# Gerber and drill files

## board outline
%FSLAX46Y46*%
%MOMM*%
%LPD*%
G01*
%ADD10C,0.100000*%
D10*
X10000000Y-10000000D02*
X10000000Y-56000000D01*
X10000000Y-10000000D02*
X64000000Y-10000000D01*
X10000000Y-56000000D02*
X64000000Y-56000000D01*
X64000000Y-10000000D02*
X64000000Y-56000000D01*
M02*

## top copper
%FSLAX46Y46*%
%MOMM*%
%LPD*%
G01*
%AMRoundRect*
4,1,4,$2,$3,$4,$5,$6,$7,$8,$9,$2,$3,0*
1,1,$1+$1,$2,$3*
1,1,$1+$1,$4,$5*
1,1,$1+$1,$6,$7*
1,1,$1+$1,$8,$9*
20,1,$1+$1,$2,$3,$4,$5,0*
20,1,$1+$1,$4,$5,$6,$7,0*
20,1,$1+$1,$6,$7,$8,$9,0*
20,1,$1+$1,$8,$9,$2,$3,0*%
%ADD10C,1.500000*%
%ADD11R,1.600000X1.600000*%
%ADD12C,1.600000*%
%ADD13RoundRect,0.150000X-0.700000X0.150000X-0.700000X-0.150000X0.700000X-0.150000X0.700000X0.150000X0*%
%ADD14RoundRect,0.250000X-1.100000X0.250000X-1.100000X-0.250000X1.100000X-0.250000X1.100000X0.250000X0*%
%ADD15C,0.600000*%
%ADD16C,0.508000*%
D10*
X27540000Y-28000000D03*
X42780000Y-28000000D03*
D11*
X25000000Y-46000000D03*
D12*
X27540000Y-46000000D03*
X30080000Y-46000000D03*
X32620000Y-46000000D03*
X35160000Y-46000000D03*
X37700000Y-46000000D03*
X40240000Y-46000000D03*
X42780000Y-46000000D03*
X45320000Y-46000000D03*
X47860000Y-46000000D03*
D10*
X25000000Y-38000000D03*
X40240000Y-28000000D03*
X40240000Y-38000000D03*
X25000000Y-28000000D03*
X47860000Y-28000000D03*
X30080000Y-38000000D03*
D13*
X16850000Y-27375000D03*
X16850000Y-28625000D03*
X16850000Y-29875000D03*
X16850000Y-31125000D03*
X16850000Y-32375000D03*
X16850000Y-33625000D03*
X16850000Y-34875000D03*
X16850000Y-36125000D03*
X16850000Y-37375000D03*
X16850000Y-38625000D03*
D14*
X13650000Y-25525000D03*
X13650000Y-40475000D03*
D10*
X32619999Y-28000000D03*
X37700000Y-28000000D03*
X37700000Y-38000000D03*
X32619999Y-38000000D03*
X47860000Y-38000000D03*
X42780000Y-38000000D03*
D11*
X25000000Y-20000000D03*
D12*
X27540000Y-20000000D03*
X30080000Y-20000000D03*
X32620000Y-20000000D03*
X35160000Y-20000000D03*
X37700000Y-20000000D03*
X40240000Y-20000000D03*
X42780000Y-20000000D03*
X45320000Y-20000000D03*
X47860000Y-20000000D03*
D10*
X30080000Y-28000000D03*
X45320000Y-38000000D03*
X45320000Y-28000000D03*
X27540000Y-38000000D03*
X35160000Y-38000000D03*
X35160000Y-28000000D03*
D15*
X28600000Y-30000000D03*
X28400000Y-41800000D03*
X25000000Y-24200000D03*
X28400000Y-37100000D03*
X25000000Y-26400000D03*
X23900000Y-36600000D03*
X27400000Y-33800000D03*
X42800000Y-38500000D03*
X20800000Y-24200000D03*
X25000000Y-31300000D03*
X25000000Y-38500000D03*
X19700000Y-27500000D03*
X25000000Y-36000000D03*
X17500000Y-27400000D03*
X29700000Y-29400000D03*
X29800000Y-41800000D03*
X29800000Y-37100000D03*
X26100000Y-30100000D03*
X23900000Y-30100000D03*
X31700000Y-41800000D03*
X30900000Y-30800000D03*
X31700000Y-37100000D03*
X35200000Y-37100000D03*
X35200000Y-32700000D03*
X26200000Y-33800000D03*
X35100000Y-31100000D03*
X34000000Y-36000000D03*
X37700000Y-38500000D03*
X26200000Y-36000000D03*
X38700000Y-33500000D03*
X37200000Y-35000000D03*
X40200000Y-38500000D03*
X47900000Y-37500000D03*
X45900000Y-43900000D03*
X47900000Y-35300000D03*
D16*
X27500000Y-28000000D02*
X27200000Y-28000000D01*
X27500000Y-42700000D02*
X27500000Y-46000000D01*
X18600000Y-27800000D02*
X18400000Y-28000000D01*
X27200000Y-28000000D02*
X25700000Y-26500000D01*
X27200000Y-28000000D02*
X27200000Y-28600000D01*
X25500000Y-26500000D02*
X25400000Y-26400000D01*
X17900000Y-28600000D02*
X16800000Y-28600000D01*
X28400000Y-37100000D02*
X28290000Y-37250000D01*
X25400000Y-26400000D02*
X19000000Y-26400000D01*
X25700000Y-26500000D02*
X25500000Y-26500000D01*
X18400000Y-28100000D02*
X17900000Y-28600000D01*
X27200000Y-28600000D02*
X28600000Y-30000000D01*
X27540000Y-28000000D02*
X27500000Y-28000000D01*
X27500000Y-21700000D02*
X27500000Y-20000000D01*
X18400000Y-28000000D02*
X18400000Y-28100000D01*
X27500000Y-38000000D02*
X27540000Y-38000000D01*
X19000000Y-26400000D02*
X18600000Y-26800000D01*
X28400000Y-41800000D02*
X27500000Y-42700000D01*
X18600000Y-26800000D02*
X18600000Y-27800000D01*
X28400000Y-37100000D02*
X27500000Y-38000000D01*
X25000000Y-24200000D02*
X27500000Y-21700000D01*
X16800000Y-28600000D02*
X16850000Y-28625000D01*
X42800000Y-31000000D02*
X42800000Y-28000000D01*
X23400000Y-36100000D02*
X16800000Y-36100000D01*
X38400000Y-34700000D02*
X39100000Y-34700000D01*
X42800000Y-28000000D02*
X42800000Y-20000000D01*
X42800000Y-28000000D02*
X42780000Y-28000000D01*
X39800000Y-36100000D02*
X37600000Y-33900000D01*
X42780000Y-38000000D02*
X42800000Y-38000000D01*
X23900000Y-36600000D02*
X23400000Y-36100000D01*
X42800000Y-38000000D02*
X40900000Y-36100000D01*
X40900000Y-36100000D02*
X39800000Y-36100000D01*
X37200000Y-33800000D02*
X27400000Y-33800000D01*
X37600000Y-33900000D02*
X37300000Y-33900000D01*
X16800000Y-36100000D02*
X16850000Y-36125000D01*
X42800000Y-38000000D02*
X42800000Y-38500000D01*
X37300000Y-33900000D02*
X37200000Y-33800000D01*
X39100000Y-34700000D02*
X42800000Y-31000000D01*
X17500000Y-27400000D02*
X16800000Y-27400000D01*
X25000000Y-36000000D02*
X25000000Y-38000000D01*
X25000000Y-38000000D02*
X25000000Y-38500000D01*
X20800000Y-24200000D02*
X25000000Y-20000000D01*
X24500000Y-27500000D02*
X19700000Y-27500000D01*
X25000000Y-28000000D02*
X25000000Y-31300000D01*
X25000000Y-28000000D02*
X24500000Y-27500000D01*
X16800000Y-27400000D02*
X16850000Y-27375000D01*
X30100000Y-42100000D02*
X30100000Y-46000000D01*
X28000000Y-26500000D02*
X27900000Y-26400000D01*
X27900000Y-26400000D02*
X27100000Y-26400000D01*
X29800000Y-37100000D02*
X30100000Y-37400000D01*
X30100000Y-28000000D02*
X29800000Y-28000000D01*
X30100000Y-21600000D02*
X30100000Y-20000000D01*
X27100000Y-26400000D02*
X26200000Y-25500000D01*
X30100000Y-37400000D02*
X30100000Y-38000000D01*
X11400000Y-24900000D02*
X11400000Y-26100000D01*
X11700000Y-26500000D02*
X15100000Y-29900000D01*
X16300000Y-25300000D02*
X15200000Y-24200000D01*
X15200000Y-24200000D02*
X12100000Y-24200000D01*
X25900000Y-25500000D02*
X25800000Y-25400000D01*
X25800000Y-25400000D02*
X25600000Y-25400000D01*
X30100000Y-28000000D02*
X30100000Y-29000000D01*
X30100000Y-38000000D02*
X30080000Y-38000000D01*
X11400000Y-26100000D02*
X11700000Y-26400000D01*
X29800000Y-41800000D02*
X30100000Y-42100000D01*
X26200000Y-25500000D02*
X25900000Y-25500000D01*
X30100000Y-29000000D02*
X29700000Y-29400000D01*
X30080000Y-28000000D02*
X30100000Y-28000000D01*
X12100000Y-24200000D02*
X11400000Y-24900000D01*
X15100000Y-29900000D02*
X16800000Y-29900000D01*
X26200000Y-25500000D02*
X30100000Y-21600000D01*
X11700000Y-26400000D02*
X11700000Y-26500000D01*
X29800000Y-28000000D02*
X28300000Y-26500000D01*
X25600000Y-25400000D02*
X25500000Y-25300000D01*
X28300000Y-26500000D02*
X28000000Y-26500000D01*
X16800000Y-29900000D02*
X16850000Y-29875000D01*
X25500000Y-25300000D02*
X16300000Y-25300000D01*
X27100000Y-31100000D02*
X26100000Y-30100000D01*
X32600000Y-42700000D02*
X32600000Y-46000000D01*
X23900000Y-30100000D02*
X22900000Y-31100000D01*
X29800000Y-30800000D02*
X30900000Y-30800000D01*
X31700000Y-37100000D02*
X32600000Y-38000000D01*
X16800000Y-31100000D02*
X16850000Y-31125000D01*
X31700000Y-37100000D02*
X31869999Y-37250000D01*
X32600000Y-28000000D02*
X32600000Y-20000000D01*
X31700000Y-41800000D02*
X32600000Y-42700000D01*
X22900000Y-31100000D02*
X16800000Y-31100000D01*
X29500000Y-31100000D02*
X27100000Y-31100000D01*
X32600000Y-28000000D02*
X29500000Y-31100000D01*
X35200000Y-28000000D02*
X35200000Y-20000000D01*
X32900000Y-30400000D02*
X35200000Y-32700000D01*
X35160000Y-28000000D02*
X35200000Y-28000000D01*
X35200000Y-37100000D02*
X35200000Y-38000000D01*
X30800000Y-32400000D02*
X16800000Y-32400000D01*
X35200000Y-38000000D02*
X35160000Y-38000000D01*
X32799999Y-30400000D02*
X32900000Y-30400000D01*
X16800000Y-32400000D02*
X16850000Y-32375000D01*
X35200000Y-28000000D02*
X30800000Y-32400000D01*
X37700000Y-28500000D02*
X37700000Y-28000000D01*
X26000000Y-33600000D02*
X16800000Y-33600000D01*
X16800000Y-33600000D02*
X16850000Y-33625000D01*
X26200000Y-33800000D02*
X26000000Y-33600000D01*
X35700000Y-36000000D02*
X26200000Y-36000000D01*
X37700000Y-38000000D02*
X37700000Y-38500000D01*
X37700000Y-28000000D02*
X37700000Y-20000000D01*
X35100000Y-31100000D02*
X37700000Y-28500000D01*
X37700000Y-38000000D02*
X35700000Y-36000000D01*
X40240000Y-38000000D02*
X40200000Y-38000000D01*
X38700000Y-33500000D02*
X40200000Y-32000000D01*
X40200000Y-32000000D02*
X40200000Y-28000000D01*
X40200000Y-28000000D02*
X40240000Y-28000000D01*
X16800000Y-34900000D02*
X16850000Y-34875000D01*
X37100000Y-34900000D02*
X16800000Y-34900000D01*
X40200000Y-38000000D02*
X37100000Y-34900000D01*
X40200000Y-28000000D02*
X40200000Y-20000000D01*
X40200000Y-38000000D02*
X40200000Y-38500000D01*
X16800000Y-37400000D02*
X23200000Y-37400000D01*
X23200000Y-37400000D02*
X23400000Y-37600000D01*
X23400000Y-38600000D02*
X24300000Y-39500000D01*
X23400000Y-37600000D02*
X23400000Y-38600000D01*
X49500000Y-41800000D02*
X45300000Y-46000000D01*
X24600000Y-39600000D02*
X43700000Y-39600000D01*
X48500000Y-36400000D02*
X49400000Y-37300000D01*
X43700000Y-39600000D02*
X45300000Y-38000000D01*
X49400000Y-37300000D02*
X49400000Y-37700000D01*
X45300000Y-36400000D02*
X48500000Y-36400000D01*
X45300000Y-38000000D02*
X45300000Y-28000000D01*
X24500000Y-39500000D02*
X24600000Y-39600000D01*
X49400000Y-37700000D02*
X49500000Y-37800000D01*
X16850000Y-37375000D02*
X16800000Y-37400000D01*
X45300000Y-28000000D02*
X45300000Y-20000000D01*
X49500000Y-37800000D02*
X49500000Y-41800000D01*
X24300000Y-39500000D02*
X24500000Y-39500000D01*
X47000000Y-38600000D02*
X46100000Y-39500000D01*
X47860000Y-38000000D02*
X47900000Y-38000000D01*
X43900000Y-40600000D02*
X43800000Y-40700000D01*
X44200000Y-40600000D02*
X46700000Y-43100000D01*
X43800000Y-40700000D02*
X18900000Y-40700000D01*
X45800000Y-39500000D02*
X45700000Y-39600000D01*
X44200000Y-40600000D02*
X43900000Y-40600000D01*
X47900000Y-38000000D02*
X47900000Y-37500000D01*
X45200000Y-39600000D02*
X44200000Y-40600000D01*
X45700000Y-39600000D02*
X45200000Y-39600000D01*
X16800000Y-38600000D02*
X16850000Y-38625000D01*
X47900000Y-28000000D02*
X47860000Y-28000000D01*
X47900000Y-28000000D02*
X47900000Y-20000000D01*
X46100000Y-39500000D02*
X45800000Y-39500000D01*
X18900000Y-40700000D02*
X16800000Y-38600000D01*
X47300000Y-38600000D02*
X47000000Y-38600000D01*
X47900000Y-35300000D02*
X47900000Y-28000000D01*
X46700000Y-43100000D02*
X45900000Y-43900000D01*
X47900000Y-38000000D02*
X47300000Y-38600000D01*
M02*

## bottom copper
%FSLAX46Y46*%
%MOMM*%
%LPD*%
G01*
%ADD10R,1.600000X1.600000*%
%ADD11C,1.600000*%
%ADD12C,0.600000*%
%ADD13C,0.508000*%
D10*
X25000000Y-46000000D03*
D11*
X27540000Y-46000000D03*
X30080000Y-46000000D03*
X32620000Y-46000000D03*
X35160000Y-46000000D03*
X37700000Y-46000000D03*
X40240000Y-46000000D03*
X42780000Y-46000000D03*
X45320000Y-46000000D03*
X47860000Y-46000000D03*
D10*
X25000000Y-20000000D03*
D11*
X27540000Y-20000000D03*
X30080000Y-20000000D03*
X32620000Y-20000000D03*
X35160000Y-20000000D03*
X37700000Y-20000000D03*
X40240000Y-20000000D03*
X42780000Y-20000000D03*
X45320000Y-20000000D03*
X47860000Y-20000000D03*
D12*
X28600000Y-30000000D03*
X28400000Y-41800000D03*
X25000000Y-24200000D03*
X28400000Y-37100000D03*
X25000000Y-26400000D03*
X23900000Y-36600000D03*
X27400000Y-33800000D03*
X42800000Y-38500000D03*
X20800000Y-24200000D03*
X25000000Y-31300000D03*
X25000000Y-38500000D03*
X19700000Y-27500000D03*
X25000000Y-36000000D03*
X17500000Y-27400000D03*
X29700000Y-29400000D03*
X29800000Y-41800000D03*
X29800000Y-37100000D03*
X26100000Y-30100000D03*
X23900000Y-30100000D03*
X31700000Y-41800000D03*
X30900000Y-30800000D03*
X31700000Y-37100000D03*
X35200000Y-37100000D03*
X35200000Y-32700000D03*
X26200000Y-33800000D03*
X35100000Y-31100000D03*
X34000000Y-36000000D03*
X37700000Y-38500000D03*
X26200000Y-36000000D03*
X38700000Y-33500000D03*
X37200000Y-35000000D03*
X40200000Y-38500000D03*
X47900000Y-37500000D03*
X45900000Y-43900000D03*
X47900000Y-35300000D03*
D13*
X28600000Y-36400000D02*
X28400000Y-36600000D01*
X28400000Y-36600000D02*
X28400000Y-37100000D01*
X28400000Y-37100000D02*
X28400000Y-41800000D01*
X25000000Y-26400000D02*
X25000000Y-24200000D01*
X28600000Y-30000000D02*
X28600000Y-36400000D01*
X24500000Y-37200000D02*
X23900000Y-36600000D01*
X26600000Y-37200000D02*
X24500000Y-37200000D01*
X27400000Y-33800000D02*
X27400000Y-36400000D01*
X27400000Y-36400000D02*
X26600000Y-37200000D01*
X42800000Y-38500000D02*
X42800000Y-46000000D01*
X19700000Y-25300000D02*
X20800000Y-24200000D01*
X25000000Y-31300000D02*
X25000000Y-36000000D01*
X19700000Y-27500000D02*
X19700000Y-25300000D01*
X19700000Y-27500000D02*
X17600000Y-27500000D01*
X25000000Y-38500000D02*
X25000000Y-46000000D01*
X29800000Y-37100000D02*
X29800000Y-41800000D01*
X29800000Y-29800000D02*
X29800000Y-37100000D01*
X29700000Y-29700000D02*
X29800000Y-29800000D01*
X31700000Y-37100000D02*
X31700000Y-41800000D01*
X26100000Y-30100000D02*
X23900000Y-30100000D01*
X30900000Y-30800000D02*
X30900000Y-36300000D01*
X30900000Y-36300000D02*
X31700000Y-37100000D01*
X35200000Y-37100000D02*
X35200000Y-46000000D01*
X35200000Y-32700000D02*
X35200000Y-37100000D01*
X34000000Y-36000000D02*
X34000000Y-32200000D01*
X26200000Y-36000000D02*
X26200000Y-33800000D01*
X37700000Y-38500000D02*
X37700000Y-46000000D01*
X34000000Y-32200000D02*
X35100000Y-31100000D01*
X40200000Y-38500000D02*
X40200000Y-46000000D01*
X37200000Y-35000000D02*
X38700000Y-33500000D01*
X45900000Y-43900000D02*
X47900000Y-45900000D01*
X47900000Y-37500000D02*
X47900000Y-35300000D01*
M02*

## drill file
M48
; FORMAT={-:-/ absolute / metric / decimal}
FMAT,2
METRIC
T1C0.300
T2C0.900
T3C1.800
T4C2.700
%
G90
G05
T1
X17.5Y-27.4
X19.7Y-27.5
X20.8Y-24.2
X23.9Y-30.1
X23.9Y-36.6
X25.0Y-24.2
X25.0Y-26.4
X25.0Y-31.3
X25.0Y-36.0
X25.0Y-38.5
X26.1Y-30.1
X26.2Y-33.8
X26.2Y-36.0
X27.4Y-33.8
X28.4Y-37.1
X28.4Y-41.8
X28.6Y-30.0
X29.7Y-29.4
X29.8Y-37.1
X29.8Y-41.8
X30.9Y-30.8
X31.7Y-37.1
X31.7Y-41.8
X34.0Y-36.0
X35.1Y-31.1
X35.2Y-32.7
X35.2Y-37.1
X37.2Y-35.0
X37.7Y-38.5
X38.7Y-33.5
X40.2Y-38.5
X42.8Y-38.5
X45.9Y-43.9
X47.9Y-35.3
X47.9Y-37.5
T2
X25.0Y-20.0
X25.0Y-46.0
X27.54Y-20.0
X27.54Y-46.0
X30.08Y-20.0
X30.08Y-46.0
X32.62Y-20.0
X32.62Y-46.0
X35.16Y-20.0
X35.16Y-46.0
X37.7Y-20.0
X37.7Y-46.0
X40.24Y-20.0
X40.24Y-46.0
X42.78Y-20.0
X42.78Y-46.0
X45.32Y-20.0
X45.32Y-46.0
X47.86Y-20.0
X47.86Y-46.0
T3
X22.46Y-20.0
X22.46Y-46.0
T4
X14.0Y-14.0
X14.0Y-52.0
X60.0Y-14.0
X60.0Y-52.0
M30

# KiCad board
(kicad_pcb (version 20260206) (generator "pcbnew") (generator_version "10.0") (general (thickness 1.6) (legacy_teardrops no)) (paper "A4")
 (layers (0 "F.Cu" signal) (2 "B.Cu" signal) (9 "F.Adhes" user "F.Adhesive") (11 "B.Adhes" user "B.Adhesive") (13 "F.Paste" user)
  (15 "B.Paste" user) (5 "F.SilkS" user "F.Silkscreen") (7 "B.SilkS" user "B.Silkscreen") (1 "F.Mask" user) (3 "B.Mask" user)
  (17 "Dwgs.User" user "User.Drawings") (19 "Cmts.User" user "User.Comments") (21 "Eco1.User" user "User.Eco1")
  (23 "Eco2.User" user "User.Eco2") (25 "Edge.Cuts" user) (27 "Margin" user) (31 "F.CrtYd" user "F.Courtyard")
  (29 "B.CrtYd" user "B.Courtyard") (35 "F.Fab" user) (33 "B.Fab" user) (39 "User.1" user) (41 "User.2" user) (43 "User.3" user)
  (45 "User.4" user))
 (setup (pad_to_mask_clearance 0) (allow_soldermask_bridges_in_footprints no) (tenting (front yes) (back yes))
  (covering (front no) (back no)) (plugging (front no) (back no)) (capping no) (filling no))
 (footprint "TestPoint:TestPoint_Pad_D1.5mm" (layer "F.Cu") (at 27.54 28)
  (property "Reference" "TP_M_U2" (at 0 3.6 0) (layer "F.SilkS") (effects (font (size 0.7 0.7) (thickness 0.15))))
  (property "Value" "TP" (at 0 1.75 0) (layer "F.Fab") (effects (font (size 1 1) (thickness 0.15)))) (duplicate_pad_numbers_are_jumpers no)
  (pad "1" smd circle (at 0 0) (size 1.5 1.5) (layers "F.Cu" "F.Mask") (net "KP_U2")))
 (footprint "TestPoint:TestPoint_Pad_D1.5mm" (layer "F.Cu") (at 42.78 28)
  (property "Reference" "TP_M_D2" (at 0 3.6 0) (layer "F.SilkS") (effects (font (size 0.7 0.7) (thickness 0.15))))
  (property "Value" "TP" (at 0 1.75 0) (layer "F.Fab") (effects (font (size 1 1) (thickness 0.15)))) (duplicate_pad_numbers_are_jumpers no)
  (pad "1" smd circle (at 0 0) (size 1.5 1.5) (layers "F.Cu" "F.Mask") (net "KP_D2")))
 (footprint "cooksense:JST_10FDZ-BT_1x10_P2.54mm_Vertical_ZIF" (layer "F.Cu") (at 25 46)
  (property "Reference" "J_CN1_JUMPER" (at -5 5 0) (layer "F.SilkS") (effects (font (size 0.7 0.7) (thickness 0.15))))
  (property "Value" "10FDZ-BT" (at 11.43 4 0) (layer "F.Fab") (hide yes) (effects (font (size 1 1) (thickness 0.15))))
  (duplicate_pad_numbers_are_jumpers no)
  (pad "" np_thru_hole circle (at -2.54 0) (size 1.8 1.8) (drill 1.8) (layers "*.Cu" "*.Mask"))
  (pad "1" thru_hole rect (at 0 0) (size 1.6 1.6) (drill 0.9) (layers "*.Cu" "*.Mask") (remove_unused_layers no) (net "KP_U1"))
  (pad "2" thru_hole circle (at 2.54 0) (size 1.6 1.6) (drill 0.9) (layers "*.Cu" "*.Mask") (remove_unused_layers no) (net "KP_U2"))
  (pad "3" thru_hole circle (at 5.08 0) (size 1.6 1.6) (drill 0.9) (layers "*.Cu" "*.Mask") (remove_unused_layers no) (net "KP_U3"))
  (pad "4" thru_hole circle (at 7.62 0) (size 1.6 1.6) (drill 0.9) (layers "*.Cu" "*.Mask") (remove_unused_layers no) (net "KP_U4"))
  (pad "5" thru_hole circle (at 10.16 0) (size 1.6 1.6) (drill 0.9) (layers "*.Cu" "*.Mask") (remove_unused_layers no) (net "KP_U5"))
  (pad "6" thru_hole circle (at 12.7 0) (size 1.6 1.6) (drill 0.9) (layers "*.Cu" "*.Mask") (remove_unused_layers no) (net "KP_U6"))
  (pad "7" thru_hole circle (at 15.24 0) (size 1.6 1.6) (drill 0.9) (layers "*.Cu" "*.Mask") (remove_unused_layers no) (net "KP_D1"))
  (pad "8" thru_hole circle (at 17.78 0) (size 1.6 1.6) (drill 0.9) (layers "*.Cu" "*.Mask") (remove_unused_layers no) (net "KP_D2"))
  (pad "9" thru_hole circle (at 20.32 0) (size 1.6 1.6) (drill 0.9) (layers "*.Cu" "*.Mask") (remove_unused_layers no) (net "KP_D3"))
  (pad "10" thru_hole circle (at 22.86 0) (size 1.6 1.6) (drill 0.9) (layers "*.Cu" "*.Mask") (remove_unused_layers no) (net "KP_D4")))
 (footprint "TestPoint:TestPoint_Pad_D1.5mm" (layer "F.Cu") (at 25 38)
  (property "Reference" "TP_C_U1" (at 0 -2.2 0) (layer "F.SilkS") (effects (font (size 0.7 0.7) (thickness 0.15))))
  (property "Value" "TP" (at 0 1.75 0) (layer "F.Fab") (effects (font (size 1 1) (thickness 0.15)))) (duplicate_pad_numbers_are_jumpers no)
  (pad "1" smd circle (at 0 0) (size 1.5 1.5) (layers "F.Cu" "F.Mask") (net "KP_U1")))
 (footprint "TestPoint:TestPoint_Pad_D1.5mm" (layer "F.Cu") (at 40.24 28)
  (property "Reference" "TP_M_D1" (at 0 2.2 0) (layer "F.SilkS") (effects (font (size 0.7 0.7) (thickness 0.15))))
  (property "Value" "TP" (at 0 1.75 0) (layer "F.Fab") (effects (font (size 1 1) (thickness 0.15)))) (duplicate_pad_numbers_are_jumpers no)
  (pad "1" smd circle (at 0 0) (size 1.5 1.5) (layers "F.Cu" "F.Mask") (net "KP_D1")))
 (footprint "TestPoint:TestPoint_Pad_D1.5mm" (layer "F.Cu") (at 40.24 38)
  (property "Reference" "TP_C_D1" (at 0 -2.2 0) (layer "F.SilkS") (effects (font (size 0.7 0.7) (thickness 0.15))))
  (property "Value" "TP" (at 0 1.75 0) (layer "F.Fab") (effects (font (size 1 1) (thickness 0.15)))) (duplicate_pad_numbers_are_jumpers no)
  (pad "1" smd circle (at 0 0) (size 1.5 1.5) (layers "F.Cu" "F.Mask") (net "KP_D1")))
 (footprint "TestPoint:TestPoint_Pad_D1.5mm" (layer "F.Cu") (at 25 28)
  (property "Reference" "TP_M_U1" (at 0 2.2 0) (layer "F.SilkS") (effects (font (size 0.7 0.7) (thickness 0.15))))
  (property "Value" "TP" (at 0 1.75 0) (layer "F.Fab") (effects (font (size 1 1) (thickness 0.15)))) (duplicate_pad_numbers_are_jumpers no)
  (pad "1" smd circle (at 0 0) (size 1.5 1.5) (layers "F.Cu" "F.Mask") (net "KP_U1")))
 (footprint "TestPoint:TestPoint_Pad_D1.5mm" (layer "F.Cu") (at 47.86 28)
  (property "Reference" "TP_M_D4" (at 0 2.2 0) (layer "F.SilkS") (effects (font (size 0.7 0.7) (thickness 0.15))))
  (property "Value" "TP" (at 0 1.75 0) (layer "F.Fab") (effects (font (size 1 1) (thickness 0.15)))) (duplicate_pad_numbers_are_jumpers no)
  (pad "1" smd circle (at 0 0) (size 1.5 1.5) (layers "F.Cu" "F.Mask") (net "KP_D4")))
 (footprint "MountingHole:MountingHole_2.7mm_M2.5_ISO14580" (layer "F.Cu") (at 60 14)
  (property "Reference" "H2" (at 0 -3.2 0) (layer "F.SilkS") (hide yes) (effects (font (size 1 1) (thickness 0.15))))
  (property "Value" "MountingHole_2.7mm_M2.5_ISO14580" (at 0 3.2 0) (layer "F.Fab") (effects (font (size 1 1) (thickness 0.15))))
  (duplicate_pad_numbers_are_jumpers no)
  (pad "" np_thru_hole circle (at 0 0) (size 2.7 2.7) (drill 2.7) (layers "*.Cu" "*.Mask")))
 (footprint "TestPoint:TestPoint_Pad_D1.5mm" (layer "F.Cu") (at 30.08 38)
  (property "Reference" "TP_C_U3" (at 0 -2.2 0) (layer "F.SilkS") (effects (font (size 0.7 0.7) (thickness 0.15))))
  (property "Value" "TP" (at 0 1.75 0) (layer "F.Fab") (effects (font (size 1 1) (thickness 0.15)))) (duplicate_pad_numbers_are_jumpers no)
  (pad "1" smd circle (at 0 0) (size 1.5 1.5) (layers "F.Cu" "F.Mask") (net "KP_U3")))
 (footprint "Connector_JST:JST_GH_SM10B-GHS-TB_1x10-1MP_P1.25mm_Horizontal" (layer "F.Cu") (at 15 33 -90)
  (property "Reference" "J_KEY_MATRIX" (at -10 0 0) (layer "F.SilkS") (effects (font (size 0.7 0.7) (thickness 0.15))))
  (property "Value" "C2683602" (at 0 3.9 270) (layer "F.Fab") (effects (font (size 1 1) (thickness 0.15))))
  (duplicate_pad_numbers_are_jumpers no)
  (pad "1" smd roundrect (at -5.625 -1.85 270) (size 0.6 1.7) (layers "F.Cu" "F.Mask" "F.Paste") (roundrect_rratio 0.25) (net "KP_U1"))
  (pad "2" smd roundrect (at -4.375 -1.85 270) (size 0.6 1.7) (layers "F.Cu" "F.Mask" "F.Paste") (roundrect_rratio 0.25) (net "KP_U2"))
  (pad "3" smd roundrect (at -3.125 -1.85 270) (size 0.6 1.7) (layers "F.Cu" "F.Mask" "F.Paste") (roundrect_rratio 0.25) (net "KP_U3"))
  (pad "4" smd roundrect (at -1.875 -1.85 270) (size 0.6 1.7) (layers "F.Cu" "F.Mask" "F.Paste") (roundrect_rratio 0.25) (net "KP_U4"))
  (pad "5" smd roundrect (at -0.625 -1.85 270) (size 0.6 1.7) (layers "F.Cu" "F.Mask" "F.Paste") (roundrect_rratio 0.25) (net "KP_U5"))
  (pad "6" smd roundrect (at 0.625 -1.85 270) (size 0.6 1.7) (layers "F.Cu" "F.Mask" "F.Paste") (roundrect_rratio 0.25) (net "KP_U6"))
  (pad "7" smd roundrect (at 1.875 -1.85 270) (size 0.6 1.7) (layers "F.Cu" "F.Mask" "F.Paste") (roundrect_rratio 0.25) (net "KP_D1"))
  (pad "8" smd roundrect (at 3.125 -1.85 270) (size 0.6 1.7) (layers "F.Cu" "F.Mask" "F.Paste") (roundrect_rratio 0.25) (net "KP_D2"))
  (pad "9" smd roundrect (at 4.375 -1.85 270) (size 0.6 1.7) (layers "F.Cu" "F.Mask" "F.Paste") (roundrect_rratio 0.25) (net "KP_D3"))
  (pad "10" smd roundrect (at 5.625 -1.85 270) (size 0.6 1.7) (layers "F.Cu" "F.Mask" "F.Paste") (roundrect_rratio 0.25) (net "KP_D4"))
  (pad "MP" smd roundrect (at -7.475 1.35 270) (size 1 2.7) (layers "F.Cu" "F.Mask" "F.Paste") (roundrect_rratio 0.25))
  (pad "MP" smd roundrect (at 7.475 1.35 270) (size 1 2.7) (layers "F.Cu" "F.Mask" "F.Paste") (roundrect_rratio 0.25)))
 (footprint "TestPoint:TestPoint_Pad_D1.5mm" (layer "F.Cu") (at 32.619999 28)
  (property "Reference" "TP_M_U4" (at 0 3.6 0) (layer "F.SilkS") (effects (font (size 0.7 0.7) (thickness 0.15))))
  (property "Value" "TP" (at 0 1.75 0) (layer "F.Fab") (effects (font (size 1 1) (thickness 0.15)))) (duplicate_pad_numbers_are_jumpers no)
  (pad "1" smd circle (at 0 0) (size 1.5 1.5) (layers "F.Cu" "F.Mask") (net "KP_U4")))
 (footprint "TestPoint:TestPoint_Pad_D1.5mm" (layer "F.Cu") (at 37.7 28)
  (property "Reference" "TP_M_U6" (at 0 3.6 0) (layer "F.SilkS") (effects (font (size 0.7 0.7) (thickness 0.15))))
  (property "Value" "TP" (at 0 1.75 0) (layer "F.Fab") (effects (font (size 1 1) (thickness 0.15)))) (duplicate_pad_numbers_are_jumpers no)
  (pad "1" smd circle (at 0 0) (size 1.5 1.5) (layers "F.Cu" "F.Mask") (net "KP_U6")))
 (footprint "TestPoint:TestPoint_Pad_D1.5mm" (layer "F.Cu") (at 37.7 38)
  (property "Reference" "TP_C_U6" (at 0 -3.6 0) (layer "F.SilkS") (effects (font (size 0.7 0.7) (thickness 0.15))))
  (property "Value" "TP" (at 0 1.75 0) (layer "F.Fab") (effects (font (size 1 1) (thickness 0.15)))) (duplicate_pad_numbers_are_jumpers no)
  (pad "1" smd circle (at 0 0) (size 1.5 1.5) (layers "F.Cu" "F.Mask") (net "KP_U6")))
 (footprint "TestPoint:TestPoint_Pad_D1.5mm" (layer "F.Cu") (at 32.619999 38)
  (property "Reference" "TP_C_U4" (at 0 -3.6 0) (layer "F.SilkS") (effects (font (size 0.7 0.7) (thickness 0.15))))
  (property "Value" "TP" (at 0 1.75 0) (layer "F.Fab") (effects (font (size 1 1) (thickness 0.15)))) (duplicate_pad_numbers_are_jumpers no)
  (pad "1" smd circle (at 0 0) (size 1.5 1.5) (layers "F.Cu" "F.Mask") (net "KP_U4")))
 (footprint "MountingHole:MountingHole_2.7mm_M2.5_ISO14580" (layer "F.Cu") (at 14 14)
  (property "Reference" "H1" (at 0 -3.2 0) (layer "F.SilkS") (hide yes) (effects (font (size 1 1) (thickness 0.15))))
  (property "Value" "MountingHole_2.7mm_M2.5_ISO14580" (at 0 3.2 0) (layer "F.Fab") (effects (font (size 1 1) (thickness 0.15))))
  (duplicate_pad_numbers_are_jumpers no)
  (pad "" np_thru_hole circle (at 0 0) (size 2.7 2.7) (drill 2.7) (layers "*.Cu" "*.Mask")))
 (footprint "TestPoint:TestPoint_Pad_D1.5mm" (layer "F.Cu") (at 47.86 38)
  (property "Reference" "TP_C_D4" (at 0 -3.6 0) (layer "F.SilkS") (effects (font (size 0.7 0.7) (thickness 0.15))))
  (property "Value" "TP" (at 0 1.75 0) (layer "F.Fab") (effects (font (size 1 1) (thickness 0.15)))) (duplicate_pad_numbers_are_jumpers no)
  (pad "1" smd circle (at 0 0) (size 1.5 1.5) (layers "F.Cu" "F.Mask") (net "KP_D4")))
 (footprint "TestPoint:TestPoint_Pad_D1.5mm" (layer "F.Cu") (at 42.78 38)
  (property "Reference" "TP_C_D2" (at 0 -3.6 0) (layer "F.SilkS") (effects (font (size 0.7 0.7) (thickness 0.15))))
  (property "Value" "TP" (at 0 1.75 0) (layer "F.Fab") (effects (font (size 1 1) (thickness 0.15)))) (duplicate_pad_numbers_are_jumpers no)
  (pad "1" smd circle (at 0 0) (size 1.5 1.5) (layers "F.Cu" "F.Mask") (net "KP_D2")))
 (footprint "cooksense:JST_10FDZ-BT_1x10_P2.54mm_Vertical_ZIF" (layer "F.Cu") (at 25 20)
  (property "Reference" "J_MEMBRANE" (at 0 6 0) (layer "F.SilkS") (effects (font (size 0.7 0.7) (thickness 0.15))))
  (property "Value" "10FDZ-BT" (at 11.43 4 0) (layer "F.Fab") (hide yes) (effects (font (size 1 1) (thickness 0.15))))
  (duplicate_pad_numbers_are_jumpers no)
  (pad "" np_thru_hole circle (at -2.54 0) (size 1.8 1.8) (drill 1.8) (layers "*.Cu" "*.Mask"))
  (pad "1" thru_hole rect (at 0 0) (size 1.6 1.6) (drill 0.9) (layers "*.Cu" "*.Mask") (remove_unused_layers no) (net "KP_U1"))
  (pad "2" thru_hole circle (at 2.54 0) (size 1.6 1.6) (drill 0.9) (layers "*.Cu" "*.Mask") (remove_unused_layers no) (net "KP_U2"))
  (pad "3" thru_hole circle (at 5.08 0) (size 1.6 1.6) (drill 0.9) (layers "*.Cu" "*.Mask") (remove_unused_layers no) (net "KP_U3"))
  (pad "4" thru_hole circle (at 7.62 0) (size 1.6 1.6) (drill 0.9) (layers "*.Cu" "*.Mask") (remove_unused_layers no) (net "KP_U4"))
  (pad "5" thru_hole circle (at 10.16 0) (size 1.6 1.6) (drill 0.9) (layers "*.Cu" "*.Mask") (remove_unused_layers no) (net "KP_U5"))
  (pad "6" thru_hole circle (at 12.7 0) (size 1.6 1.6) (drill 0.9) (layers "*.Cu" "*.Mask") (remove_unused_layers no) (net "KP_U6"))
  (pad "7" thru_hole circle (at 15.24 0) (size 1.6 1.6) (drill 0.9) (layers "*.Cu" "*.Mask") (remove_unused_layers no) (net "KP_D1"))
  (pad "8" thru_hole circle (at 17.78 0) (size 1.6 1.6) (drill 0.9) (layers "*.Cu" "*.Mask") (remove_unused_layers no) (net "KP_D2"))
  (pad "9" thru_hole circle (at 20.32 0) (size 1.6 1.6) (drill 0.9) (layers "*.Cu" "*.Mask") (remove_unused_layers no) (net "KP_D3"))
  (pad "10" thru_hole circle (at 22.86 0) (size 1.6 1.6) (drill 0.9) (layers "*.Cu" "*.Mask") (remove_unused_layers no) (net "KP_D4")))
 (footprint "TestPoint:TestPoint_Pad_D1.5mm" (layer "F.Cu") (at 30.08 28)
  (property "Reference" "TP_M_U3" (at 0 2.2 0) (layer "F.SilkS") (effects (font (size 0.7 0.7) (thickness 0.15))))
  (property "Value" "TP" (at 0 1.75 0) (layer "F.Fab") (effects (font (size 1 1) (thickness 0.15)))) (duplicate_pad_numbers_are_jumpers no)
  (pad "1" smd circle (at 0 0) (size 1.5 1.5) (layers "F.Cu" "F.Mask") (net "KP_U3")))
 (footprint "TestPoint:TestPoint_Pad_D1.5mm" (layer "F.Cu") (at 45.32 38)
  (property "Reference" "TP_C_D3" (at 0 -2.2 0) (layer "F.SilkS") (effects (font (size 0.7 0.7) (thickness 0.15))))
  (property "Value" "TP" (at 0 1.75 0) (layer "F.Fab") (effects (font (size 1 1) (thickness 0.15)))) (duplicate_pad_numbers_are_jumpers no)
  (pad "1" smd circle (at 0 0) (size 1.5 1.5) (layers "F.Cu" "F.Mask") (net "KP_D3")))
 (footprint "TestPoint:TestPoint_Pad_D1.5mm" (layer "F.Cu") (at 45.32 28)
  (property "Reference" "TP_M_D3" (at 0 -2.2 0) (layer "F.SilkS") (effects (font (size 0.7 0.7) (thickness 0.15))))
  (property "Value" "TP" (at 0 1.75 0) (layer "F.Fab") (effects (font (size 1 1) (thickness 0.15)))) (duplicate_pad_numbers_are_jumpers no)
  (pad "1" smd circle (at 0 0) (size 1.5 1.5) (layers "F.Cu" "F.Mask") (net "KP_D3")))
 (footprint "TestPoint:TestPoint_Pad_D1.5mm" (layer "F.Cu") (at 27.54 38)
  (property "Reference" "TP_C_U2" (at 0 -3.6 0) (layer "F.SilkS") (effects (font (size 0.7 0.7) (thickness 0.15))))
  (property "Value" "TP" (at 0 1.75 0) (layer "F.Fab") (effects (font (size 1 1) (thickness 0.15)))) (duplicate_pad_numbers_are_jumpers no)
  (pad "1" smd circle (at 0 0) (size 1.5 1.5) (layers "F.Cu" "F.Mask") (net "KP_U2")))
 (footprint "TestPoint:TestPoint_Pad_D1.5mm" (layer "F.Cu") (at 35.16 38)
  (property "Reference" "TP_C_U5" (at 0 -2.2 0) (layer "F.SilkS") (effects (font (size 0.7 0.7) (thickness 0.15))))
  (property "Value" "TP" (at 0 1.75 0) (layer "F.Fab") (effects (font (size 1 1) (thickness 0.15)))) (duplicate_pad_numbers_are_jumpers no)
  (pad "1" smd circle (at 0 0) (size 1.5 1.5) (layers "F.Cu" "F.Mask") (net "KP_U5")))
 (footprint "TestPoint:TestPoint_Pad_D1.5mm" (layer "F.Cu") (at 35.16 28)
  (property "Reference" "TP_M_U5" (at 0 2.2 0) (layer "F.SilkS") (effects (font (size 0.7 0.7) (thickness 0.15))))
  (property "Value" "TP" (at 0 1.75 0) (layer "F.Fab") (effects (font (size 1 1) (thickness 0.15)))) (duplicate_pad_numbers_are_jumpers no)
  (pad "1" smd circle (at 0 0) (size 1.5 1.5) (layers "F.Cu" "F.Mask") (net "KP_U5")))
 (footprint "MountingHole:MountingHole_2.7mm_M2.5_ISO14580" (layer "F.Cu") (at 60 52)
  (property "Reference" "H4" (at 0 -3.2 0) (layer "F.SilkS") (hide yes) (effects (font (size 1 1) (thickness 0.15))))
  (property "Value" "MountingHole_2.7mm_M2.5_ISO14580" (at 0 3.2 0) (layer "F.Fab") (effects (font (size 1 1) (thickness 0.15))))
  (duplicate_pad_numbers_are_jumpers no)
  (pad "" np_thru_hole circle (at 0 0) (size 2.7 2.7) (drill 2.7) (layers "*.Cu" "*.Mask")))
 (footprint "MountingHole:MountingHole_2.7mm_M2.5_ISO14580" (layer "F.Cu") (at 14 52)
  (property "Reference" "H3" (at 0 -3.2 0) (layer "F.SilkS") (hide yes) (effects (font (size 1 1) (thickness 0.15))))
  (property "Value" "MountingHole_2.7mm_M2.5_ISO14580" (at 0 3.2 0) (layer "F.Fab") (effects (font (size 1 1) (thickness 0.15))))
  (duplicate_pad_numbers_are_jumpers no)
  (pad "" np_thru_hole circle (at 0 0) (size 2.7 2.7) (drill 2.7) (layers "*.Cu" "*.Mask")))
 (gr_line (start 10 10) (end 10 56) (stroke (width 0.1) (type default)) (layer "Edge.Cuts"))
 (gr_line (start 10 10) (end 64 10) (stroke (width 0.1) (type default)) (layer "Edge.Cuts"))
 (gr_line (start 10 56) (end 64 56) (stroke (width 0.1) (type default)) (layer "Edge.Cuts"))
 (gr_line (start 64 10) (end 64 56) (stroke (width 0.1) (type default)) (layer "Edge.Cuts"))
 (segment (start 27.5 28) (end 27.2 28) (width 0.508) (layer "F.Cu") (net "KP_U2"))
 (segment (start 27.5 42.7) (end 27.5 46) (width 0.508) (layer "F.Cu") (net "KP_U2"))
 (segment (start 18.6 27.8) (end 18.4 28) (width 0.508) (layer "F.Cu") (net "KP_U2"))
 (segment (start 27.2 28) (end 25.7 26.5) (width 0.508) (layer "F.Cu") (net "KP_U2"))
 (segment (start 27.2 28) (end 27.2 28.6) (width 0.508) (layer "F.Cu") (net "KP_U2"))
 (segment (start 25.5 26.5) (end 25.4 26.4) (width 0.508) (layer "F.Cu") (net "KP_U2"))
 (segment (start 17.9 28.6) (end 16.8 28.6) (width 0.508) (layer "F.Cu") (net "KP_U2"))
 (segment (start 28.4 37.1) (end 28.29 37.25) (width 0.508) (layer "F.Cu") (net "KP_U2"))
 (segment (start 25.4 26.4) (end 19 26.4) (width 0.508) (layer "F.Cu") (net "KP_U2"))
 (segment (start 25.7 26.5) (end 25.5 26.5) (width 0.508) (layer "F.Cu") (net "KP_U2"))
 (segment (start 18.4 28.1) (end 17.9 28.6) (width 0.508) (layer "F.Cu") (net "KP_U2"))
 (segment (start 27.2 28.6) (end 28.6 30) (width 0.508) (layer "F.Cu") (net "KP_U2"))
 (segment (start 27.54 28) (end 27.5 28) (width 0.508) (layer "F.Cu") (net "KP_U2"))
 (segment (start 27.5 21.7) (end 27.5 20) (width 0.508) (layer "F.Cu") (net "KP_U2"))
 (segment (start 18.4 28) (end 18.4 28.1) (width 0.508) (layer "F.Cu") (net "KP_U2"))
 (segment (start 27.5 38) (end 27.54 38) (width 0.508) (layer "F.Cu") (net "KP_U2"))
 (segment (start 19 26.4) (end 18.6 26.8) (width 0.508) (layer "F.Cu") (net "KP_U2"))
 (segment (start 28.4 41.8) (end 27.5 42.7) (width 0.508) (layer "F.Cu") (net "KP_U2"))
 (segment (start 18.6 26.8) (end 18.6 27.8) (width 0.508) (layer "F.Cu") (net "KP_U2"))
 (segment (start 28.4 37.1) (end 27.5 38) (width 0.508) (layer "F.Cu") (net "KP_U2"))
 (segment (start 25 24.2) (end 27.5 21.7) (width 0.508) (layer "F.Cu") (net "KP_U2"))
 (segment (start 16.8 28.6) (end 16.85 28.625) (width 0.508) (layer "F.Cu") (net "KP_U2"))
 (via (at 28.6 30) (size 0.6) (drill 0.3) (layers "F.Cu" "B.Cu") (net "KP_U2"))
 (via (at 28.4 41.8) (size 0.6) (drill 0.3) (layers "F.Cu" "B.Cu") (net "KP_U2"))
 (via (at 25 24.2) (size 0.6) (drill 0.3) (layers "F.Cu" "B.Cu") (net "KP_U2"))
 (via (at 28.4 37.1) (size 0.6) (drill 0.3) (layers "F.Cu" "B.Cu") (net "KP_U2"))
 (via (at 25 26.4) (size 0.6) (drill 0.3) (layers "F.Cu" "B.Cu") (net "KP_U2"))
 (segment (start 28.6 36.4) (end 28.4 36.6) (width 0.508) (layer "B.Cu") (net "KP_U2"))
 (segment (start 28.4 36.6) (end 28.4 37.1) (width 0.508) (layer "B.Cu") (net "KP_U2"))
 (segment (start 28.4 37.1) (end 28.4 41.8) (width 0.508) (layer "B.Cu") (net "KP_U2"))
 (segment (start 25 26.4) (end 25 24.2) (width 0.508) (layer "B.Cu") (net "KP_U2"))
 (segment (start 28.6 30) (end 28.6 36.4) (width 0.508) (layer "B.Cu") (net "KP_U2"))
 (segment (start 42.8 31) (end 42.8 28) (width 0.508) (layer "F.Cu") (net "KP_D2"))
 (segment (start 23.4 36.1) (end 16.8 36.1) (width 0.508) (layer "F.Cu") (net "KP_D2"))
 (segment (start 38.4 34.7) (end 39.1 34.7) (width 0.508) (layer "F.Cu") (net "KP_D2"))
 (segment (start 42.8 28) (end 42.8 20) (width 0.508) (layer "F.Cu") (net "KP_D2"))
 (segment (start 42.8 28) (end 42.78 28) (width 0.508) (layer "F.Cu") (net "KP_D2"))
 (segment (start 39.8 36.1) (end 37.6 33.9) (width 0.508) (layer "F.Cu") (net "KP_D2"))
 (segment (start 42.78 38) (end 42.8 38) (width 0.508) (layer "F.Cu") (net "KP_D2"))
 (segment (start 23.9 36.6) (end 23.4 36.1) (width 0.508) (layer "F.Cu") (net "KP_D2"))
 (segment (start 42.8 38) (end 40.9 36.1) (width 0.508) (layer "F.Cu") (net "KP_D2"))
 (segment (start 40.9 36.1) (end 39.8 36.1) (width 0.508) (layer "F.Cu") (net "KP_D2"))
 (segment (start 37.2 33.8) (end 27.4 33.8) (width 0.508) (layer "F.Cu") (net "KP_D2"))
 (segment (start 37.6 33.9) (end 37.3 33.9) (width 0.508) (layer "F.Cu") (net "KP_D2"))
 (segment (start 16.8 36.1) (end 16.85 36.125) (width 0.508) (layer "F.Cu") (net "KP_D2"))
 (segment (start 42.8 38) (end 42.8 38.5) (width 0.508) (layer "F.Cu") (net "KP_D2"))
 (segment (start 37.3 33.9) (end 37.2 33.8) (width 0.508) (layer "F.Cu") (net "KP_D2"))
 (segment (start 39.1 34.7) (end 42.8 31) (width 0.508) (layer "F.Cu") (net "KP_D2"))
 (via (at 23.9 36.6) (size 0.6) (drill 0.3) (layers "F.Cu" "B.Cu") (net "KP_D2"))
 (via (at 27.4 33.8) (size 0.6) (drill 0.3) (layers "F.Cu" "B.Cu") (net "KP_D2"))
 (via (at 42.8 38.5) (size 0.6) (drill 0.3) (layers "F.Cu" "B.Cu") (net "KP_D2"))
 (segment (start 24.5 37.2) (end 23.9 36.6) (width 0.508) (layer "B.Cu") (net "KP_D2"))
 (segment (start 26.6 37.2) (end 24.5 37.2) (width 0.508) (layer "B.Cu") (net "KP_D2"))
 (segment (start 27.4 33.8) (end 27.4 36.4) (width 0.508) (layer "B.Cu") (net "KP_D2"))
 (segment (start 27.4 36.4) (end 26.6 37.2) (width 0.508) (layer "B.Cu") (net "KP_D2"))
 (segment (start 42.8 38.5) (end 42.8 46) (width 0.508) (layer "B.Cu") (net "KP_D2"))
 (segment (start 17.5 27.4) (end 16.8 27.4) (width 0.508) (layer "F.Cu") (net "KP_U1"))
 (segment (start 25 36) (end 25 38) (width 0.508) (layer "F.Cu") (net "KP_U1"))
 (segment (start 25 38) (end 25 38.5) (width 0.508) (layer "F.Cu") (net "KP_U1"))
 (segment (start 20.8 24.2) (end 25 20) (width 0.508) (layer "F.Cu") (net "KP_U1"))
 (segment (start 24.5 27.5) (end 19.7 27.5) (width 0.508) (layer "F.Cu") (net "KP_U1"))
 (segment (start 25 28) (end 25 31.3) (width 0.508) (layer "F.Cu") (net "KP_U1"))
 (segment (start 25 28) (end 24.5 27.5) (width 0.508) (layer "F.Cu") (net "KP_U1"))
 (segment (start 16.8 27.4) (end 16.85 27.375) (width 0.508) (layer "F.Cu") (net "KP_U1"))
 (via (at 20.8 24.2) (size 0.6) (drill 0.3) (layers "F.Cu" "B.Cu") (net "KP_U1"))
 (via (at 25 31.3) (size 0.6) (drill 0.3) (layers "F.Cu" "B.Cu") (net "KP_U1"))
 (via (at 25 38.5) (size 0.6) (drill 0.3) (layers "F.Cu" "B.Cu") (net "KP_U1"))
 (via (at 19.7 27.5) (size 0.6) (drill 0.3) (layers "F.Cu" "B.Cu") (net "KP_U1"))
 (via (at 25 36) (size 0.6) (drill 0.3) (layers "F.Cu" "B.Cu") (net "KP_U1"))
 (via (at 17.5 27.4) (size 0.6) (drill 0.3) (layers "F.Cu" "B.Cu") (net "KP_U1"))
 (segment (start 19.7 25.3) (end 20.8 24.2) (width 0.508) (layer "B.Cu") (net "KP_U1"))
 (segment (start 25 31.3) (end 25 36) (width 0.508) (layer "B.Cu") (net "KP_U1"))
 (segment (start 19.7 27.5) (end 19.7 25.3) (width 0.508) (layer "B.Cu") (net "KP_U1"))
 (segment (start 19.7 27.5) (end 17.6 27.5) (width 0.508) (layer "B.Cu") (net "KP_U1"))
 (segment (start 25 38.5) (end 25 46) (width 0.508) (layer "B.Cu") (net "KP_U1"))
 (segment (start 30.1 42.1) (end 30.1 46) (width 0.508) (layer "F.Cu") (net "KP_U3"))
 (segment (start 28 26.5) (end 27.9 26.4) (width 0.508) (layer "F.Cu") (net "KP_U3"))
 (segment (start 27.9 26.4) (end 27.1 26.4) (width 0.508) (layer "F.Cu") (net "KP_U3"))
 (segment (start 29.8 37.1) (end 30.1 37.4) (width 0.508) (layer "F.Cu") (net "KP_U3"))
 (segment (start 30.1 28) (end 29.8 28) (width 0.508) (layer "F.Cu") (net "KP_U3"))
 (segment (start 30.1 21.6) (end 30.1 20) (width 0.508) (layer "F.Cu") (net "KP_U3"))
 (segment (start 27.1 26.4) (end 26.2 25.5) (width 0.508) (layer "F.Cu") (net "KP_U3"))
 (segment (start 30.1 37.4) (end 30.1 38) (width 0.508) (layer "F.Cu") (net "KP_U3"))
 (segment (start 11.4 24.9) (end 11.4 26.1) (width 0.508) (layer "F.Cu") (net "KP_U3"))
 (segment (start 11.7 26.5) (end 15.1 29.9) (width 0.508) (layer "F.Cu") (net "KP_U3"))
 (segment (start 16.3 25.3) (end 15.2 24.2) (width 0.508) (layer "F.Cu") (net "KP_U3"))
 (segment (start 15.2 24.2) (end 12.1 24.2) (width 0.508) (layer "F.Cu") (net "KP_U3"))
 (segment (start 25.9 25.5) (end 25.8 25.4) (width 0.508) (layer "F.Cu") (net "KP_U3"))
 (segment (start 25.8 25.4) (end 25.6 25.4) (width 0.508) (layer "F.Cu") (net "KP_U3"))
 (segment (start 30.1 28) (end 30.1 29) (width 0.508) (layer "F.Cu") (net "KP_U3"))
 (segment (start 30.1 38) (end 30.08 38) (width 0.508) (layer "F.Cu") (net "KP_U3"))
 (segment (start 11.4 26.1) (end 11.7 26.4) (width 0.508) (layer "F.Cu") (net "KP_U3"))
 (segment (start 29.8 41.8) (end 30.1 42.1) (width 0.508) (layer "F.Cu") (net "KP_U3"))
 (segment (start 26.2 25.5) (end 25.9 25.5) (width 0.508) (layer "F.Cu") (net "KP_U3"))
 (segment (start 30.1 29) (end 29.7 29.4) (width 0.508) (layer "F.Cu") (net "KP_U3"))
 (segment (start 30.08 28) (end 30.1 28) (width 0.508) (layer "F.Cu") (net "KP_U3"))
 (segment (start 12.1 24.2) (end 11.4 24.9) (width 0.508) (layer "F.Cu") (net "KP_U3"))
 (segment (start 15.1 29.9) (end 16.8 29.9) (width 0.508) (layer "F.Cu") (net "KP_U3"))
 (segment (start 26.2 25.5) (end 30.1 21.6) (width 0.508) (layer "F.Cu") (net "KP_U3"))
 (segment (start 11.7 26.4) (end 11.7 26.5) (width 0.508) (layer "F.Cu") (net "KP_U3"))
 (segment (start 29.8 28) (end 28.3 26.5) (width 0.508) (layer "F.Cu") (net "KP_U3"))
 (segment (start 25.6 25.4) (end 25.5 25.3) (width 0.508) (layer "F.Cu") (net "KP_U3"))
 (segment (start 28.3 26.5) (end 28 26.5) (width 0.508) (layer "F.Cu") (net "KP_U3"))
 (segment (start 16.8 29.9) (end 16.85 29.875) (width 0.508) (layer "F.Cu") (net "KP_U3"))
 (segment (start 25.5 25.3) (end 16.3 25.3) (width 0.508) (layer "F.Cu") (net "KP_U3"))
 (via (at 29.7 29.4) (size 0.6) (drill 0.3) (layers "F.Cu" "B.Cu") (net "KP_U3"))
 (via (at 29.8 41.8) (size 0.6) (drill 0.3) (layers "F.Cu" "B.Cu") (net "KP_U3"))
 (via (at 29.8 37.1) (size 0.6) (drill 0.3) (layers "F.Cu" "B.Cu") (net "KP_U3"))
 (segment (start 29.8 37.1) (end 29.8 41.8) (width 0.508) (layer "B.Cu") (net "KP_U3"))
 (segment (start 29.8 29.8) (end 29.8 37.1) (width 0.508) (layer "B.Cu") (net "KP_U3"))
 (segment (start 29.7 29.7) (end 29.8 29.8) (width 0.508) (layer "B.Cu") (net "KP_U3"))
 (segment (start 27.1 31.1) (end 26.1 30.1) (width 0.508) (layer "F.Cu") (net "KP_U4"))
 (segment (start 32.6 42.7) (end 32.6 46) (width 0.508) (layer "F.Cu") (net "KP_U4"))
 (segment (start 23.9 30.1) (end 22.9 31.1) (width 0.508) (layer "F.Cu") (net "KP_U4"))
 (segment (start 29.8 30.8) (end 30.9 30.8) (width 0.508) (layer "F.Cu") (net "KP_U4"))
 (segment (start 31.7 37.1) (end 32.6 38) (width 0.508) (layer "F.Cu") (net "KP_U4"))
 (segment (start 16.8 31.1) (end 16.85 31.125) (width 0.508) (layer "F.Cu") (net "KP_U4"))
 (segment (start 31.7 37.1) (end 31.869999 37.25) (width 0.508) (layer "F.Cu") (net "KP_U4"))
 (segment (start 32.6 28) (end 32.6 20) (width 0.508) (layer "F.Cu") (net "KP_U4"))
 (segment (start 31.7 41.8) (end 32.6 42.7) (width 0.508) (layer "F.Cu") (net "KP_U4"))
 (segment (start 22.9 31.1) (end 16.8 31.1) (width 0.508) (layer "F.Cu") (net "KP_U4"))
 (segment (start 29.5 31.1) (end 27.1 31.1) (width 0.508) (layer "F.Cu") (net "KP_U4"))
 (segment (start 32.6 28) (end 29.5 31.1) (width 0.508) (layer "F.Cu") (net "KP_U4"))
 (via (at 26.1 30.1) (size 0.6) (drill 0.3) (layers "F.Cu" "B.Cu") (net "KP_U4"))
 (via (at 23.9 30.1) (size 0.6) (drill 0.3) (layers "F.Cu" "B.Cu") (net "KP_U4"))
 (via (at 31.7 41.8) (size 0.6) (drill 0.3) (layers "F.Cu" "B.Cu") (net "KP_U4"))
 (via (at 30.9 30.8) (size 0.6) (drill 0.3) (layers "F.Cu" "B.Cu") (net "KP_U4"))
 (via (at 31.7 37.1) (size 0.6) (drill 0.3) (layers "F.Cu" "B.Cu") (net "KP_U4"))
 (segment (start 31.7 37.1) (end 31.7 41.8) (width 0.508) (layer "B.Cu") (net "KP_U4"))
 (segment (start 26.1 30.1) (end 23.9 30.1) (width 0.508) (layer "B.Cu") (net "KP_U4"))
 (segment (start 30.9 30.8) (end 30.9 36.3) (width 0.508) (layer "B.Cu") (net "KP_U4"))
 (segment (start 30.9 36.3) (end 31.7 37.1) (width 0.508) (layer "B.Cu") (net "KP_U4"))
 (segment (start 35.2 28) (end 35.2 20) (width 0.508) (layer "F.Cu") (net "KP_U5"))
 (segment (start 32.9 30.4) (end 35.2 32.7) (width 0.508) (layer "F.Cu") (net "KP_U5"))
 (segment (start 35.16 28) (end 35.2 28) (width 0.508) (layer "F.Cu") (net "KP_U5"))
 (segment (start 35.2 37.1) (end 35.2 38) (width 0.508) (layer "F.Cu") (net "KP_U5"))
 (segment (start 30.8 32.4) (end 16.8 32.4) (width 0.508) (layer "F.Cu") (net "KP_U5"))
 (segment (start 35.2 38) (end 35.16 38) (width 0.508) (layer "F.Cu") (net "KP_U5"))
 (segment (start 32.799999 30.4) (end 32.9 30.4) (width 0.508) (layer "F.Cu") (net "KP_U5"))
 (segment (start 16.8 32.4) (end 16.85 32.375) (width 0.508) (layer "F.Cu") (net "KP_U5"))
 (segment (start 35.2 28) (end 30.8 32.4) (width 0.508) (layer "F.Cu") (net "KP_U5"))
 (via (at 35.2 37.1) (size 0.6) (drill 0.3) (layers "F.Cu" "B.Cu") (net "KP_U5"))
 (via (at 35.2 32.7) (size 0.6) (drill 0.3) (layers "F.Cu" "B.Cu") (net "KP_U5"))
 (segment (start 35.2 37.1) (end 35.2 46) (width 0.508) (layer "B.Cu") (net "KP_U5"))
 (segment (start 35.2 32.7) (end 35.2 37.1) (width 0.508) (layer "B.Cu") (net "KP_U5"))
 (segment (start 37.7 28.5) (end 37.7 28) (width 0.508) (layer "F.Cu") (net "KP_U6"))
 (segment (start 26 33.6) (end 16.8 33.6) (width 0.508) (layer "F.Cu") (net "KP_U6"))
 (segment (start 16.8 33.6) (end 16.85 33.625) (width 0.508) (layer "F.Cu") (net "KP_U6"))
 (segment (start 26.2 33.8) (end 26 33.6) (width 0.508) (layer "F.Cu") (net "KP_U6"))
 (segment (start 35.7 36) (end 26.2 36) (width 0.508) (layer "F.Cu") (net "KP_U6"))
 (segment (start 37.7 38) (end 37.7 38.5) (width 0.508) (layer "F.Cu") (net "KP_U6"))
 (segment (start 37.7 28) (end 37.7 20) (width 0.508) (layer "F.Cu") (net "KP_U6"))
 (segment (start 35.1 31.1) (end 37.7 28.5) (width 0.508) (layer "F.Cu") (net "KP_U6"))
 (segment (start 37.7 38) (end 35.7 36) (width 0.508) (layer "F.Cu") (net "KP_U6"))
 (via (at 26.2 33.8) (size 0.6) (drill 0.3) (layers "F.Cu" "B.Cu") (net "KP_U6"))
 (via (at 35.1 31.1) (size 0.6) (drill 0.3) (layers "F.Cu" "B.Cu") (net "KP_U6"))
 (via (at 34 36) (size 0.6) (drill 0.3) (layers "F.Cu" "B.Cu") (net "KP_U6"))
 (via (at 37.7 38.5) (size 0.6) (drill 0.3) (layers "F.Cu" "B.Cu") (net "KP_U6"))
 (via (at 26.2 36) (size 0.6) (drill 0.3) (layers "F.Cu" "B.Cu") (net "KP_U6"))
 (segment (start 34 36) (end 34 32.2) (width 0.508) (layer "B.Cu") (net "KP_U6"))
 (segment (start 26.2 36) (end 26.2 33.8) (width 0.508) (layer "B.Cu") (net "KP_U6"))
 (segment (start 37.7 38.5) (end 37.7 46) (width 0.508) (layer "B.Cu") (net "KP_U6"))
 (segment (start 34 32.2) (end 35.1 31.1) (width 0.508) (layer "B.Cu") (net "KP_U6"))
 (segment (start 40.24 38) (end 40.2 38) (width 0.508) (layer "F.Cu") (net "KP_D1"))
 (segment (start 38.7 33.5) (end 40.2 32) (width 0.508) (layer "F.Cu") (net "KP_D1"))
 (segment (start 40.2 32) (end 40.2 28) (width 0.508) (layer "F.Cu") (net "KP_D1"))
 (segment (start 40.2 28) (end 40.24 28) (width 0.508) (layer "F.Cu") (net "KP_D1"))
 (segment (start 16.8 34.9) (end 16.85 34.875) (width 0.508) (layer "F.Cu") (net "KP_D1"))
 (segment (start 37.1 34.9) (end 16.8 34.9) (width 0.508) (layer "F.Cu") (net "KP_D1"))
 (segment (start 40.2 38) (end 37.1 34.9) (width 0.508) (layer "F.Cu") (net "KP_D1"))
 (segment (start 40.2 28) (end 40.2 20) (width 0.508) (layer "F.Cu") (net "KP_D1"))
 (segment (start 40.2 38) (end 40.2 38.5) (width 0.508) (layer "F.Cu") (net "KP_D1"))
 (via (at 38.7 33.5) (size 0.6) (drill 0.3) (layers "F.Cu" "B.Cu") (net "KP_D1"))
 (via (at 37.2 35) (size 0.6) (drill 0.3) (layers "F.Cu" "B.Cu") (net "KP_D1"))
 (via (at 40.2 38.5) (size 0.6) (drill 0.3) (layers "F.Cu" "B.Cu") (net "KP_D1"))
 (segment (start 40.2 38.5) (end 40.2 46) (width 0.508) (layer "B.Cu") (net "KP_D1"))
 (segment (start 37.2 35) (end 38.7 33.5) (width 0.508) (layer "B.Cu") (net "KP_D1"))
 (segment (start 16.8 37.4) (end 23.2 37.4) (width 0.508) (layer "F.Cu") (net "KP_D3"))
 (segment (start 23.2 37.4) (end 23.4 37.6) (width 0.508) (layer "F.Cu") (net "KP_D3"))
 (segment (start 23.4 38.6) (end 24.3 39.5) (width 0.508) (layer "F.Cu") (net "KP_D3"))
 (segment (start 23.4 37.6) (end 23.4 38.6) (width 0.508) (layer "F.Cu") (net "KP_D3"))
 (segment (start 49.5 41.8) (end 45.3 46) (width 0.508) (layer "F.Cu") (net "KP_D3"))
 (segment (start 24.6 39.6) (end 43.7 39.6) (width 0.508) (layer "F.Cu") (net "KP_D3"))
 (segment (start 48.5 36.4) (end 49.4 37.3) (width 0.508) (layer "F.Cu") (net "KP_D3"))
 (segment (start 43.7 39.6) (end 45.3 38) (width 0.508) (layer "F.Cu") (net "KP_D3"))
 (segment (start 49.4 37.3) (end 49.4 37.7) (width 0.508) (layer "F.Cu") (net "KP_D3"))
 (segment (start 45.3 36.4) (end 48.5 36.4) (width 0.508) (layer "F.Cu") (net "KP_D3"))
 (segment (start 45.3 38) (end 45.3 28) (width 0.508) (layer "F.Cu") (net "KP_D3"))
 (segment (start 24.5 39.5) (end 24.6 39.6) (width 0.508) (layer "F.Cu") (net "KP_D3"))
 (segment (start 49.4 37.7) (end 49.5 37.8) (width 0.508) (layer "F.Cu") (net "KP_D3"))
 (segment (start 16.85 37.375) (end 16.8 37.4) (width 0.508) (layer "F.Cu") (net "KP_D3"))
 (segment (start 45.3 28) (end 45.3 20) (width 0.508) (layer "F.Cu") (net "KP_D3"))
 (segment (start 49.5 37.8) (end 49.5 41.8) (width 0.508) (layer "F.Cu") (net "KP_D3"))
 (segment (start 24.3 39.5) (end 24.5 39.5) (width 0.508) (layer "F.Cu") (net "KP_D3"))
 (segment (start 47 38.6) (end 46.1 39.5) (width 0.508) (layer "F.Cu") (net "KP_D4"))
 (segment (start 47.86 38) (end 47.9 38) (width 0.508) (layer "F.Cu") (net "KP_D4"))
 (segment (start 43.9 40.6) (end 43.8 40.7) (width 0.508) (layer "F.Cu") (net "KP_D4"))
 (segment (start 44.2 40.6) (end 46.7 43.1) (width 0.508) (layer "F.Cu") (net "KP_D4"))
 (segment (start 43.8 40.7) (end 18.9 40.7) (width 0.508) (layer "F.Cu") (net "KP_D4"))
 (segment (start 45.8 39.5) (end 45.7 39.6) (width 0.508) (layer "F.Cu") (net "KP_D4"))
 (segment (start 44.2 40.6) (end 43.9 40.6) (width 0.508) (layer "F.Cu") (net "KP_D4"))
 (segment (start 47.9 38) (end 47.9 37.5) (width 0.508) (layer "F.Cu") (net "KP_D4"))
 (segment (start 45.2 39.6) (end 44.2 40.6) (width 0.508) (layer "F.Cu") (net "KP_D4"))
 (segment (start 45.7 39.6) (end 45.2 39.6) (width 0.508) (layer "F.Cu") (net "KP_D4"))
 (segment (start 16.8 38.6) (end 16.85 38.625) (width 0.508) (layer "F.Cu") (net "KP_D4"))
 (segment (start 47.9 28) (end 47.86 28) (width 0.508) (layer "F.Cu") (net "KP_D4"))
 (segment (start 47.9 28) (end 47.9 20) (width 0.508) (layer "F.Cu") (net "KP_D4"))
 (segment (start 46.1 39.5) (end 45.8 39.5) (width 0.508) (layer "F.Cu") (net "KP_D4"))
 (segment (start 18.9 40.7) (end 16.8 38.6) (width 0.508) (layer "F.Cu") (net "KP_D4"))
 (segment (start 47.3 38.6) (end 47 38.6) (width 0.508) (layer "F.Cu") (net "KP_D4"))
 (segment (start 47.9 35.3) (end 47.9 28) (width 0.508) (layer "F.Cu") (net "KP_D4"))
 (segment (start 46.7 43.1) (end 45.9 43.9) (width 0.508) (layer "F.Cu") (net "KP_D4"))
 (segment (start 47.9 38) (end 47.3 38.6) (width 0.508) (layer "F.Cu") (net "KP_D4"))
 (via (at 47.9 37.5) (size 0.6) (drill 0.3) (layers "F.Cu" "B.Cu") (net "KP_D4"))
 (via (at 45.9 43.9) (size 0.6) (drill 0.3) (layers "F.Cu" "B.Cu") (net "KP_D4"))
 (via (at 47.9 35.3) (size 0.6) (drill 0.3) (layers "F.Cu" "B.Cu") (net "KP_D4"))
 (segment (start 45.9 43.9) (end 47.9 45.9) (width 0.508) (layer "B.Cu") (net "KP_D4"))
 (segment (start 47.9 37.5) (end 47.9 35.3) (width 0.508) (layer "B.Cu") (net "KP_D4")))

